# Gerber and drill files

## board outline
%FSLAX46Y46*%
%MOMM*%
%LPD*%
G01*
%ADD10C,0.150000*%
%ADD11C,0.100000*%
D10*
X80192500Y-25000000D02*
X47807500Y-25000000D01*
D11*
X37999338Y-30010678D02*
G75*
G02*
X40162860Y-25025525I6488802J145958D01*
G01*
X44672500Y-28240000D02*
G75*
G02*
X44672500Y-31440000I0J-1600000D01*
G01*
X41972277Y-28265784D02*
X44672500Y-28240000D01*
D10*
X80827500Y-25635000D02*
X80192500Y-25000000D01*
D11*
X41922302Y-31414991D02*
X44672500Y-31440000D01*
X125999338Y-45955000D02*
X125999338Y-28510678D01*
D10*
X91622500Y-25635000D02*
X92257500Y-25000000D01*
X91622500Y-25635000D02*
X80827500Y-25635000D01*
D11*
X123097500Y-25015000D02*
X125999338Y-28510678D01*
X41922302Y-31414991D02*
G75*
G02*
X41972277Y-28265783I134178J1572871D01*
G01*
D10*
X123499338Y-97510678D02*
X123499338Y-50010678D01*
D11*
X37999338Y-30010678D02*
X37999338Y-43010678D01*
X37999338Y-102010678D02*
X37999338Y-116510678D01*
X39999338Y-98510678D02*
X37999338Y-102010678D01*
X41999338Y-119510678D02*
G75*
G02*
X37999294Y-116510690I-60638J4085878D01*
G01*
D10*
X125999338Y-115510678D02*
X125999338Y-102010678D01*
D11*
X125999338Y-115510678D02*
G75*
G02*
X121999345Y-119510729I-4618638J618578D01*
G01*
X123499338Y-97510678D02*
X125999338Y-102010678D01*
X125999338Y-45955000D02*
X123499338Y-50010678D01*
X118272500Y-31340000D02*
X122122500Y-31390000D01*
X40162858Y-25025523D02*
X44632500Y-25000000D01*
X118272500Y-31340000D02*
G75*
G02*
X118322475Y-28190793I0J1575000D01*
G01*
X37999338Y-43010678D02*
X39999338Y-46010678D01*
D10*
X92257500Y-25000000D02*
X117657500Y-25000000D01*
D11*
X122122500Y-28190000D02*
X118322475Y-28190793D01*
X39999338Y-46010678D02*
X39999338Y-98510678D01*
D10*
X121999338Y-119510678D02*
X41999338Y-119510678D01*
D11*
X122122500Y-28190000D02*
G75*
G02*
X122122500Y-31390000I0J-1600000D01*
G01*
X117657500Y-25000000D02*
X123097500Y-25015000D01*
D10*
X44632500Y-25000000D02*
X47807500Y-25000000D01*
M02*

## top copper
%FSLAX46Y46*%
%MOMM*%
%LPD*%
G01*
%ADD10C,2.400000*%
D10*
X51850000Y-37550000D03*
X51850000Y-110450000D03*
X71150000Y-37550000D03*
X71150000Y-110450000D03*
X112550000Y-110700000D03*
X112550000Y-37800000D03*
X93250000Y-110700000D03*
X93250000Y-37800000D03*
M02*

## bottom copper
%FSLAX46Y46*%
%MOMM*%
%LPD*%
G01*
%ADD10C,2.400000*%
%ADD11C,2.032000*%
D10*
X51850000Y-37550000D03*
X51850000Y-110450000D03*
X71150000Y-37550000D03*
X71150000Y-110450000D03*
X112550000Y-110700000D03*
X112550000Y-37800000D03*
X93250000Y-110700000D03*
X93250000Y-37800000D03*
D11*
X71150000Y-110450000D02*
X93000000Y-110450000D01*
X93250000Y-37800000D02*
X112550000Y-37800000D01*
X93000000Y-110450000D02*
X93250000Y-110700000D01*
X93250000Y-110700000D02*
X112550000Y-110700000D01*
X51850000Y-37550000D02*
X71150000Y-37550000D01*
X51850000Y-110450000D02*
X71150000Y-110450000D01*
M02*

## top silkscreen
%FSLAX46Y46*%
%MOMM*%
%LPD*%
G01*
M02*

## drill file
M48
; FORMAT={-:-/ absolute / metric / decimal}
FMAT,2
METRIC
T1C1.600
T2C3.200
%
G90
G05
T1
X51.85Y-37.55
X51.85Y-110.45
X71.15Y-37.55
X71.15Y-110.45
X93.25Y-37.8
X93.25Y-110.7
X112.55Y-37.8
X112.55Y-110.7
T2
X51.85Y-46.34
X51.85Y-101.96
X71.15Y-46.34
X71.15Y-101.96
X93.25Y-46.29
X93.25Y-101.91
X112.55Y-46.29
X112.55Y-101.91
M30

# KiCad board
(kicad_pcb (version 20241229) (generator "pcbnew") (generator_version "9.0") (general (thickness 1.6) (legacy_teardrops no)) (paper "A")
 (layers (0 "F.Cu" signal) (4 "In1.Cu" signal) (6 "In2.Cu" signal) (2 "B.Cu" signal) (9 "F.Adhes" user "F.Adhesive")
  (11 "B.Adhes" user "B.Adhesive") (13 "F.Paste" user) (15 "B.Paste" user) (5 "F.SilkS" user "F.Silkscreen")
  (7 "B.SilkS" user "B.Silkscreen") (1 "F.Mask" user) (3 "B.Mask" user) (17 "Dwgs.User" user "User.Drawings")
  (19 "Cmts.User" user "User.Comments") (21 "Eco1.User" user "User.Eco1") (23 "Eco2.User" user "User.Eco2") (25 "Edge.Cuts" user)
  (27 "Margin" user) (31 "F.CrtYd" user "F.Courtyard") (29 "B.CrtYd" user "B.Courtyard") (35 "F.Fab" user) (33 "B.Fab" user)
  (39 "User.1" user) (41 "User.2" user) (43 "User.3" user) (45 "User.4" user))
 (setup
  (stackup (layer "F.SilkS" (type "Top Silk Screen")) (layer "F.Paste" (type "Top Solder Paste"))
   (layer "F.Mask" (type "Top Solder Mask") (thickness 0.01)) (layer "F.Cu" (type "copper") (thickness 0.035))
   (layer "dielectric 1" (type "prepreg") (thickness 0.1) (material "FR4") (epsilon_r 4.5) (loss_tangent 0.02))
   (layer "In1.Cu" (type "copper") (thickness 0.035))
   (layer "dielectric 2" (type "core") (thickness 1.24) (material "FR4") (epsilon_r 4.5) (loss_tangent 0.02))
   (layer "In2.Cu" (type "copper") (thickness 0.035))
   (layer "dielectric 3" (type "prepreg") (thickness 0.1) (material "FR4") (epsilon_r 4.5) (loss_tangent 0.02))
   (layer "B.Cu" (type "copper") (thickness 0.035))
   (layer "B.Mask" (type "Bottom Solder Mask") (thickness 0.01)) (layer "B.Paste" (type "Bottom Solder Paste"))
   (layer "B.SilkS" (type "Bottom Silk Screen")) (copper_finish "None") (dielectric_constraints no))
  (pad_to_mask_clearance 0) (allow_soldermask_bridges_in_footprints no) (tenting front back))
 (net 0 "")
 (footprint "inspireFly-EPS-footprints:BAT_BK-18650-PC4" (layer "B.Cu") (at 61.5 74.15 -90)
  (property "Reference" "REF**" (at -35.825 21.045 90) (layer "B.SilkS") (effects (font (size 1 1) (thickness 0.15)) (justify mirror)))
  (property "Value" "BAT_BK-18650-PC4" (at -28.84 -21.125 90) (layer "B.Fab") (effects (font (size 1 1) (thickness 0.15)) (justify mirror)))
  (pad "" np_thru_hole circle (at -27.81 -9.65 270) (size 3.2 3.2) (drill 3.2) (layers "*.Cu" "*.Mask"))
  (pad "" np_thru_hole circle (at -27.81 9.65 270) (size 3.2 3.2) (drill 3.2) (layers "*.Cu" "*.Mask"))
  (pad "" np_thru_hole circle (at 27.81 -9.65 270) (size 3.2 3.2) (drill 3.2) (layers "*.Cu" "*.Mask"))
  (pad "" np_thru_hole circle (at 27.81 9.65 270) (size 3.2 3.2) (drill 3.2) (layers "*.Cu" "*.Mask"))
  (pad "1+" thru_hole circle (at -36.6 9.65 270) (size 2.4 2.4) (drill 1.6) (layers "*.Cu" "*.Mask") (remove_unused_layers no)
   (solder_mask_margin 0.102))
  (pad "1-" thru_hole circle (at 36.3 9.65 270) (size 2.4 2.4) (drill 1.6) (layers "*.Cu" "*.Mask") (remove_unused_layers no)
   (solder_mask_margin 0.102))
  (pad "2+" thru_hole circle (at -36.6 -9.65 270) (size 2.4 2.4) (drill 1.6) (layers "*.Cu" "*.Mask") (remove_unused_layers no)
   (solder_mask_margin 0.102))
  (pad "2-" thru_hole circle (at 36.3 -9.65 270) (size 2.4 2.4) (drill 1.6) (layers "*.Cu" "*.Mask") (remove_unused_layers no)
   (solder_mask_margin 0.102)))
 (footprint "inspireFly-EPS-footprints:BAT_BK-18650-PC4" (layer "B.Cu") (at 102.9 74.1 90)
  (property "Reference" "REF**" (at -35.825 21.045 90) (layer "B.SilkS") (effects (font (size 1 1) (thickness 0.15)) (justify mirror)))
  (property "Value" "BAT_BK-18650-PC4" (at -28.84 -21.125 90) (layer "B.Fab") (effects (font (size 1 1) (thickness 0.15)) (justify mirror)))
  (pad "" np_thru_hole circle (at -27.81 -9.65 90) (size 3.2 3.2) (drill 3.2) (layers "*.Cu" "*.Mask"))
  (pad "" np_thru_hole circle (at -27.81 9.65 90) (size 3.2 3.2) (drill 3.2) (layers "*.Cu" "*.Mask"))
  (pad "" np_thru_hole circle (at 27.81 -9.65 90) (size 3.2 3.2) (drill 3.2) (layers "*.Cu" "*.Mask"))
  (pad "" np_thru_hole circle (at 27.81 9.65 90) (size 3.2 3.2) (drill 3.2) (layers "*.Cu" "*.Mask"))
  (pad "1+" thru_hole circle (at -36.6 9.65 90) (size 2.4 2.4) (drill 1.6) (layers "*.Cu" "*.Mask") (remove_unused_layers no)
   (solder_mask_margin 0.102))
  (pad "1-" thru_hole circle (at 36.3 9.65 90) (size 2.4 2.4) (drill 1.6) (layers "*.Cu" "*.Mask") (remove_unused_layers no)
   (solder_mask_margin 0.102))
  (pad "2+" thru_hole circle (at -36.6 -9.65 90) (size 2.4 2.4) (drill 1.6) (layers "*.Cu" "*.Mask") (remove_unused_layers no)
   (solder_mask_margin 0.102))
  (pad "2-" thru_hole circle (at 36.3 -9.65 90) (size 2.4 2.4) (drill 1.6) (layers "*.Cu" "*.Mask") (remove_unused_layers no)
   (solder_mask_margin 0.102)))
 (gr_line (start 80.1925 25) (end 47.8075 25) (stroke (width 0.15) (type solid)) (locked yes) (layer "Edge.Cuts"))
 (gr_arc (start 37.999338 30.010678) (mid 38.53423 27.280764) (end 40.162858 25.025523) (stroke (width 0.1) (type solid)) (locked yes)
  (layer "Edge.Cuts"))
 (gr_arc (start 44.6725 28.24) (mid 46.272496 29.84) (end 44.6725 31.44) (stroke (width 0.1) (type solid)) (locked yes) (layer "Edge.Cuts"))
 (gr_line (start 41.972277 28.265784) (end 44.6725 28.24) (stroke (width 0.1) (type solid)) (locked yes) (layer "Edge.Cuts"))
 (gr_line (start 80.8275 25.635) (end 80.1925 25) (stroke (width 0.15) (type solid)) (locked yes) (layer "Edge.Cuts"))
 (gr_line (start 41.922302 31.414991) (end 44.6725 31.44) (stroke (width 0.1) (type solid)) (locked yes) (layer "Edge.Cuts"))
 (gr_line (start 125.999338 45.955) (end 125.999338 28.510678) (stroke (width 0.1) (type solid)) (locked yes) (layer "Edge.Cuts"))
 (gr_line (start 91.6225 25.635) (end 92.2575 25) (stroke (width 0.15) (type solid)) (locked yes) (layer "Edge.Cuts"))
 (gr_line (start 91.6225 25.635) (end 80.8275 25.635) (stroke (width 0.15) (type solid)) (locked yes) (layer "Edge.Cuts"))
 (gr_line (start 123.0975 25.015) (end 125.999338 28.510678) (stroke (width 0.1) (type solid)) (locked yes) (layer "Edge.Cuts"))
 (gr_arc (start 41.922302 31.414991) (mid 40.478092 29.817073) (end 41.972277 28.265784) (stroke (width 0.1) (type solid)) (locked yes)
  (layer "Edge.Cuts"))
 (gr_line (start 123.499338 97.510678) (end 123.499338 50.010678) (stroke (width 0.15) (type solid)) (locked yes) (layer "Edge.Cuts"))
 (gr_line (start 37.999338 30.010678) (end 37.999338 43.010678) (stroke (width 0.1) (type solid)) (locked yes) (layer "Edge.Cuts"))
 (gr_line (start 37.999338 102.010678) (end 37.999338 116.510678) (stroke (width 0.1) (type solid)) (locked yes) (layer "Edge.Cuts"))
 (gr_line (start 39.999338 98.510678) (end 37.999338 102.010678) (stroke (width 0.1) (type solid)) (locked yes) (layer "Edge.Cuts"))
 (gr_arc (start 41.999338 119.510678) (mid 39.486941 118.693867) (end 37.999338 116.510678) (stroke (width 0.1) (type solid)) (locked yes)
  (layer "Edge.Cuts"))
 (gr_line (start 125.999338 115.510678) (end 125.999338 102.010678) (stroke (width 0.15) (type solid)) (locked yes) (layer "Edge.Cuts"))
 (gr_arc (start 125.999338 115.510678) (mid 124.675744 118.187084) (end 121.999338 119.510678) (stroke (width 0.1) (type solid))
  (locked yes) (layer "Edge.Cuts"))
 (gr_line (start 123.499338 97.510678) (end 125.999338 102.010678) (stroke (width 0.1) (type solid)) (locked yes) (layer "Edge.Cuts"))
 (gr_line (start 125.999338 45.955) (end 123.499338 50.010678) (stroke (width 0.1) (type solid)) (locked yes) (layer "Edge.Cuts"))
 (gr_line (start 118.2725 31.34) (end 122.1225 31.39) (stroke (width 0.1) (type solid)) (locked yes) (layer "Edge.Cuts"))
 (gr_line (start 40.162858 25.025523) (end 44.6325 25) (stroke (width 0.1) (type solid)) (locked yes) (layer "Edge.Cuts"))
 (gr_arc (start 118.2725 31.34) (mid 116.697694 29.740009) (end 118.322475 28.190793) (stroke (width 0.1) (type solid)) (locked yes)
  (layer "Edge.Cuts"))
 (gr_line (start 37.999338 43.010678) (end 39.999338 46.010678) (stroke (width 0.1) (type solid)) (locked yes) (layer "Edge.Cuts"))
 (gr_line (start 92.2575 25) (end 117.6575 25) (stroke (width 0.15) (type solid)) (locked yes) (layer "Edge.Cuts"))
 (gr_line (start 122.1225 28.19) (end 118.322475 28.190793) (stroke (width 0.1) (type solid)) (locked yes) (layer "Edge.Cuts"))
 (gr_line (start 39.999338 46.010678) (end 39.999338 98.510678) (stroke (width 0.1) (type solid)) (locked yes) (layer "Edge.Cuts"))
 (gr_line (start 121.999338 119.510678) (end 41.999338 119.510678) (stroke (width 0.15) (type solid)) (locked yes) (layer "Edge.Cuts"))
 (gr_arc (start 122.1225 28.19) (mid 123.722496 29.79) (end 122.1225 31.39) (stroke (width 0.1) (type solid)) (locked yes)
  (layer "Edge.Cuts"))
 (gr_line (start 117.6575 25) (end 123.0975 25.015) (stroke (width 0.1) (type solid)) (locked yes) (layer "Edge.Cuts"))
 (gr_line (start 44.6325 25) (end 47.8075 25) (stroke (width 0.15) (type solid)) (locked yes) (layer "Edge.Cuts"))
 (segment (start 71.15 110.45) (end 93 110.45) (width 2.032) (layer "B.Cu") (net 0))
 (segment (start 93.25 37.8) (end 112.55 37.8) (width 2.032) (layer "B.Cu") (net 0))
 (segment (start 93 110.45) (end 93.25 110.7) (width 2.032) (layer "B.Cu") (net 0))
 (segment (start 93.25 110.7) (end 112.55 110.7) (width 2.032) (layer "B.Cu") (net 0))
 (segment (start 51.85 37.55) (end 71.15 37.55) (width 2.032) (layer "B.Cu") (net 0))
 (segment (start 51.85 110.45) (end 71.15 110.45) (width 2.032) (layer "B.Cu") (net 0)))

